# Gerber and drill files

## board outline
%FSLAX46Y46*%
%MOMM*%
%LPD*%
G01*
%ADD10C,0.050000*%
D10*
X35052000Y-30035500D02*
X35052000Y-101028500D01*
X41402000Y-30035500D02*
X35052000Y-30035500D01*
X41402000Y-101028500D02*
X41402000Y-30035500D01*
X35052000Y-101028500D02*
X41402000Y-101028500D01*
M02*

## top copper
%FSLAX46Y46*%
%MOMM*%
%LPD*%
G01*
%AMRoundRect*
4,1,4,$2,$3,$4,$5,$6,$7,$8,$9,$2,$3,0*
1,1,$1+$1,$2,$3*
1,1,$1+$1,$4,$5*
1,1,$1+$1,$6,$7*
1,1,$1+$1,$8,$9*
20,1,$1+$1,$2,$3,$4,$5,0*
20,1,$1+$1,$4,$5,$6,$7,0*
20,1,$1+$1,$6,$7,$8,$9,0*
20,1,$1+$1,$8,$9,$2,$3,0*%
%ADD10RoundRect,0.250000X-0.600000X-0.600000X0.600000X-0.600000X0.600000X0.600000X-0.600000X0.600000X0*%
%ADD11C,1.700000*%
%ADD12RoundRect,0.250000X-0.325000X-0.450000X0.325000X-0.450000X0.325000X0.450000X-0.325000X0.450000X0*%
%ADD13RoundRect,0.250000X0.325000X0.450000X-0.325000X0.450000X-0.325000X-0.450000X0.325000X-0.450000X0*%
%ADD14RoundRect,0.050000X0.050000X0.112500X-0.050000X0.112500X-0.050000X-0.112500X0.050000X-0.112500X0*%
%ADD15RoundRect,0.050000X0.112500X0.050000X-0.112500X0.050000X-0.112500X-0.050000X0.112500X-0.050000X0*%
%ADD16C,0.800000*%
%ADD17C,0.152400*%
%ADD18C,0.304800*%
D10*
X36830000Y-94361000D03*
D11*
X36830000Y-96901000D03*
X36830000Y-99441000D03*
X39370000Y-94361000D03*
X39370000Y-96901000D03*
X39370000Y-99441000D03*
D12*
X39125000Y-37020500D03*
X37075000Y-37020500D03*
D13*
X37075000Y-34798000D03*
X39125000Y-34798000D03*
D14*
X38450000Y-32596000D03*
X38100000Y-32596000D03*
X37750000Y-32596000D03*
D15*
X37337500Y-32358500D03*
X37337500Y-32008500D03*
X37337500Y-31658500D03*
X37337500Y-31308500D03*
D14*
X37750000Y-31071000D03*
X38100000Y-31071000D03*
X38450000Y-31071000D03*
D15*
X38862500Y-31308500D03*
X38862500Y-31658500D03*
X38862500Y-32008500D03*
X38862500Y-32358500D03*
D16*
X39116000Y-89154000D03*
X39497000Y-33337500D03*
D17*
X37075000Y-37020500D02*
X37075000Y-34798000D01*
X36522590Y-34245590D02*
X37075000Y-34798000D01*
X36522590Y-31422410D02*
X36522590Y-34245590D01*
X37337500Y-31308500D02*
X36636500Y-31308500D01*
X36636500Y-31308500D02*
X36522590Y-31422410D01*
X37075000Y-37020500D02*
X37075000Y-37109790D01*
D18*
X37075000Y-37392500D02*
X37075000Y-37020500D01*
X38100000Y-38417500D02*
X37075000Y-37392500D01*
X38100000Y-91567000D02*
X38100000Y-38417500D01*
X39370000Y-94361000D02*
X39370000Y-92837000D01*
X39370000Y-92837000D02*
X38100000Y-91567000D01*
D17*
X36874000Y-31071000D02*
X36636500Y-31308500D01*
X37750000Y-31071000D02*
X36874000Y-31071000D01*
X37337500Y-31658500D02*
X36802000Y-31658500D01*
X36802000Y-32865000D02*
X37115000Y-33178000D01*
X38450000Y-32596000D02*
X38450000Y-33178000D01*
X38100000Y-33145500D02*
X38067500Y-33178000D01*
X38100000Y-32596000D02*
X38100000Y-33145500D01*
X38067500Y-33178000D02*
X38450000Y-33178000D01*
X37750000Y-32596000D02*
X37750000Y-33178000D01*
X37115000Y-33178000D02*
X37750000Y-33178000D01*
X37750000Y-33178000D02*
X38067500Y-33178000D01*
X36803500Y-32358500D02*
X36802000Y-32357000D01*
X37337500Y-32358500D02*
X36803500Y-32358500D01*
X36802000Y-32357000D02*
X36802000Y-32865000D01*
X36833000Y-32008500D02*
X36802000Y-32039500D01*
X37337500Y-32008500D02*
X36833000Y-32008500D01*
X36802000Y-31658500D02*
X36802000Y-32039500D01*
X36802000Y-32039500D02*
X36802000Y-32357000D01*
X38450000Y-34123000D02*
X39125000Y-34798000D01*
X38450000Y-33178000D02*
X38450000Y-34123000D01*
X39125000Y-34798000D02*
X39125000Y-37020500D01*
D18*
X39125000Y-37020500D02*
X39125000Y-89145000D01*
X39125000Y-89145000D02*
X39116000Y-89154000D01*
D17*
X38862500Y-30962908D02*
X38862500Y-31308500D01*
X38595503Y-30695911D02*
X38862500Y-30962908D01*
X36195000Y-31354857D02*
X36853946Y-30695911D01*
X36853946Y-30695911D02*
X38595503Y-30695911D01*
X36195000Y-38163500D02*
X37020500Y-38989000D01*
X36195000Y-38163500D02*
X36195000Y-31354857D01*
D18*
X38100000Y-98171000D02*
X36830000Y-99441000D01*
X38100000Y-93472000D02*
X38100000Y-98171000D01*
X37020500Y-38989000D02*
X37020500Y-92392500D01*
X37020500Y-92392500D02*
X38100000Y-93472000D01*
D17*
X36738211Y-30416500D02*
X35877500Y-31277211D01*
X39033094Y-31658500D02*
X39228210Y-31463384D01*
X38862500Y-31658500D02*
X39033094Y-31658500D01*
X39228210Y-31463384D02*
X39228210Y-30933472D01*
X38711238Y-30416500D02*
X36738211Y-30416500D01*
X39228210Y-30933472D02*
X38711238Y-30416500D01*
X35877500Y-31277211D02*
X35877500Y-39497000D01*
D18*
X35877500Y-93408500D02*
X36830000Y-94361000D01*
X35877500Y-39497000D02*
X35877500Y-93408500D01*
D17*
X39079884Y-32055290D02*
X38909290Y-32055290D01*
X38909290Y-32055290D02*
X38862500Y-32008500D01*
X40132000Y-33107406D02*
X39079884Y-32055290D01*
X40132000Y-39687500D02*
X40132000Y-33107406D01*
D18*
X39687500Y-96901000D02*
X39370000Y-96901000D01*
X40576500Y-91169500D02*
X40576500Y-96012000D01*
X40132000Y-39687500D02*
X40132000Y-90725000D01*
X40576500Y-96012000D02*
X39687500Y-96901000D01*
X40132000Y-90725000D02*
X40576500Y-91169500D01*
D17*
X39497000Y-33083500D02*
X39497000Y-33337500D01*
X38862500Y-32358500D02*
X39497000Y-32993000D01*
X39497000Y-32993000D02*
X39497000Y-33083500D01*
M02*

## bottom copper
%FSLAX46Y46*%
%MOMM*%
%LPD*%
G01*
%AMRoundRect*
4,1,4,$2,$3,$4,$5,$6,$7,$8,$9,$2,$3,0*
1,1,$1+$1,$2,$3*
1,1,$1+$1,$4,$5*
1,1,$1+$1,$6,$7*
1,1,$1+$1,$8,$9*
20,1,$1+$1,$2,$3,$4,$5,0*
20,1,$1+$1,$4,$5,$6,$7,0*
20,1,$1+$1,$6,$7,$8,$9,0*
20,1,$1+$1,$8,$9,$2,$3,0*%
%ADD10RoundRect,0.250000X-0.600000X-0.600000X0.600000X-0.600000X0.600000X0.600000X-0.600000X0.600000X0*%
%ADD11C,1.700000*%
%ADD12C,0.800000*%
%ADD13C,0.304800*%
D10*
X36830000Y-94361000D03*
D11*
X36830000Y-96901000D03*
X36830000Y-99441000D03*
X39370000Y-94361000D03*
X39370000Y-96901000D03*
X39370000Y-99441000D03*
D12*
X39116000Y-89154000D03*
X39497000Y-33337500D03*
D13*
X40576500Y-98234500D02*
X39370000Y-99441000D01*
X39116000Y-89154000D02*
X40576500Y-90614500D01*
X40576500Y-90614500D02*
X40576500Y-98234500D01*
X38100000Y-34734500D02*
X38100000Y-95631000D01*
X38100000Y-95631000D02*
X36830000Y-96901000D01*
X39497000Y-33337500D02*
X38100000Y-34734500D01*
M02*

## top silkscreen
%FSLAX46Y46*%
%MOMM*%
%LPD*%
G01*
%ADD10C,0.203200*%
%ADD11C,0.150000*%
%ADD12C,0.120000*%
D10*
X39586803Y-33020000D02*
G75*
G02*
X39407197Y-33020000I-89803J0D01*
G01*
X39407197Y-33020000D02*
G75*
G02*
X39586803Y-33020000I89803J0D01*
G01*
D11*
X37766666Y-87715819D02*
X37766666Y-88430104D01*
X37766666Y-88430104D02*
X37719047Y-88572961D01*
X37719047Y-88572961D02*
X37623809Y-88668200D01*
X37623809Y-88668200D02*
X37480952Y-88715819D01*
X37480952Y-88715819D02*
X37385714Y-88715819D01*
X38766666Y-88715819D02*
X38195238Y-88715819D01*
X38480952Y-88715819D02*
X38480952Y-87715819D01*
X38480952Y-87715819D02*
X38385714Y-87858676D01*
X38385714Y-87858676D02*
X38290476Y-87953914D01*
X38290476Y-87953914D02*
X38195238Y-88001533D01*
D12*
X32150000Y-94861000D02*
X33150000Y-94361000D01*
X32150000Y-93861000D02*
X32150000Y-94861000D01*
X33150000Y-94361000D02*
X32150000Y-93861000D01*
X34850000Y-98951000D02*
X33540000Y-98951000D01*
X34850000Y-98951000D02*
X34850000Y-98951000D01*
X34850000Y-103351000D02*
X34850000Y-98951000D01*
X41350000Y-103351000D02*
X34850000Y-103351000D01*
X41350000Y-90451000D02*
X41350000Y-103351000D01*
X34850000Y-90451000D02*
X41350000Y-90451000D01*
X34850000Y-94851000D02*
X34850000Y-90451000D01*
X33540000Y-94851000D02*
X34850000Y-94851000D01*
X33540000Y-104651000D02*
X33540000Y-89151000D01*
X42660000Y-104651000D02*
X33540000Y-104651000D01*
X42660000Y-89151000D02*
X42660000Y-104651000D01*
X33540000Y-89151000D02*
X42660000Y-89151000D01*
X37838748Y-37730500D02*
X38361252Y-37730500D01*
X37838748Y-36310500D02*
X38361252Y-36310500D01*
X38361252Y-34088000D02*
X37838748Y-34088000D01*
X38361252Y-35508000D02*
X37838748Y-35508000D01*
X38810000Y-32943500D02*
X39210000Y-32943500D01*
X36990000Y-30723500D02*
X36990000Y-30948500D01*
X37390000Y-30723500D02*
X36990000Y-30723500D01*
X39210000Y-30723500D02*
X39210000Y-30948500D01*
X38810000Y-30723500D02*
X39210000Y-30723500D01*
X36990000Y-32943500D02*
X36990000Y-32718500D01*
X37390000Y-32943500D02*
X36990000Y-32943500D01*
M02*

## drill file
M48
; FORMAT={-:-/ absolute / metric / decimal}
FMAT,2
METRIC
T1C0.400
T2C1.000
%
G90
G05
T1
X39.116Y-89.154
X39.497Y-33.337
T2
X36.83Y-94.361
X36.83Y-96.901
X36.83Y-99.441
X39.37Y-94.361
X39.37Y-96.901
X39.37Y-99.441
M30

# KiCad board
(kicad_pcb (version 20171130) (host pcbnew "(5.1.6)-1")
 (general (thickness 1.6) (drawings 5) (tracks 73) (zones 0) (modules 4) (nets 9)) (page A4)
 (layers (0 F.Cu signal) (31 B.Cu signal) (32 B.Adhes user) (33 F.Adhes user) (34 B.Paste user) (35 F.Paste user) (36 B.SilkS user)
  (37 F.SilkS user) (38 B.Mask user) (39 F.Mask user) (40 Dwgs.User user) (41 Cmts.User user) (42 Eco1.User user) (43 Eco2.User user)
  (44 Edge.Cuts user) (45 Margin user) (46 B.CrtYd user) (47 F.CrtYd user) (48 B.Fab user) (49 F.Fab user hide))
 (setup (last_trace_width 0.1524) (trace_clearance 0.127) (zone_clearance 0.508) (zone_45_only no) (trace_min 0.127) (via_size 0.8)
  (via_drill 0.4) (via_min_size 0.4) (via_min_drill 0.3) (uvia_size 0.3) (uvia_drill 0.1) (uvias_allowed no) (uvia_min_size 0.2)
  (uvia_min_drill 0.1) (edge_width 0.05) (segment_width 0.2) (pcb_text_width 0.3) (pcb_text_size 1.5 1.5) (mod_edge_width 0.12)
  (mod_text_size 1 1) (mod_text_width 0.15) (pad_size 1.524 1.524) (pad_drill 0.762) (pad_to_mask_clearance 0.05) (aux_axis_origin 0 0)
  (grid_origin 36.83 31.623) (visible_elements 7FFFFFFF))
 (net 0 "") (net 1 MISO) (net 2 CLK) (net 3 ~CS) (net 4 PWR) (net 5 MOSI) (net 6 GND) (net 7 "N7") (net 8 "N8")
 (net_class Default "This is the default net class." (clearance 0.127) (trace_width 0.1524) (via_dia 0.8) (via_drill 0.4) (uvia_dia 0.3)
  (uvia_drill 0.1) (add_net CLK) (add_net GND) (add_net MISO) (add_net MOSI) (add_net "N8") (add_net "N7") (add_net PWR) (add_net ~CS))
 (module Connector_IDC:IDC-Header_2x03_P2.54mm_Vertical (layer F.Cu) (at 36.83 94.361)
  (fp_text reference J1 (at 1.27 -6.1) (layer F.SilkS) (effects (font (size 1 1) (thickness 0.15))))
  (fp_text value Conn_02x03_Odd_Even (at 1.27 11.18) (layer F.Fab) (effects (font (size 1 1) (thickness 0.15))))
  (fp_line (start -4.68 0.5) (end -3.68 0) (layer F.SilkS) (width 0.12))
  (fp_line (start -4.68 -0.5) (end -4.68 0.5) (layer F.SilkS) (width 0.12))
  (fp_line (start -3.68 0) (end -4.68 -0.5) (layer F.SilkS) (width 0.12))
  (fp_line (start -1.98 4.59) (end -3.29 4.59) (layer F.SilkS) (width 0.12))
  (fp_line (start -1.98 4.59) (end -1.98 4.59) (layer F.SilkS) (width 0.12))
  (fp_line (start -1.98 8.99) (end -1.98 4.59) (layer F.SilkS) (width 0.12))
  (fp_line (start 4.52 8.99) (end -1.98 8.99) (layer F.SilkS) (width 0.12))
  (fp_line (start 4.52 -3.91) (end 4.52 8.99) (layer F.SilkS) (width 0.12))
  (fp_line (start -1.98 -3.91) (end 4.52 -3.91) (layer F.SilkS) (width 0.12))
  (fp_line (start -1.98 0.49) (end -1.98 -3.91) (layer F.SilkS) (width 0.12))
  (fp_line (start -3.29 0.49) (end -1.98 0.49) (layer F.SilkS) (width 0.12))
  (fp_line (start -3.29 10.29) (end -3.29 -5.21) (layer F.SilkS) (width 0.12))
  (fp_line (start 5.83 10.29) (end -3.29 10.29) (layer F.SilkS) (width 0.12))
  (fp_line (start 5.83 -5.21) (end 5.83 10.29) (layer F.SilkS) (width 0.12))
  (fp_line (start -3.29 -5.21) (end 5.83 -5.21) (layer F.SilkS) (width 0.12))
  (pad 1 thru_hole roundrect (at 0 0) (size 1.7 1.7) (drill 1) (layers *.Cu *.Mask) (roundrect_rratio 0.147059) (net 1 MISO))
  (pad 3 thru_hole circle (at 0 2.54) (size 1.7 1.7) (drill 1) (layers *.Cu *.Mask) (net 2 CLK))
  (pad 5 thru_hole circle (at 0 5.08) (size 1.7 1.7) (drill 1) (layers *.Cu *.Mask) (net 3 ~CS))
  (pad 2 thru_hole circle (at 2.54 0) (size 1.7 1.7) (drill 1) (layers *.Cu *.Mask) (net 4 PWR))
  (pad 4 thru_hole circle (at 2.54 2.54) (size 1.7 1.7) (drill 1) (layers *.Cu *.Mask) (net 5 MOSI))
  (pad 6 thru_hole circle (at 2.54 5.08) (size 1.7 1.7) (drill 1) (layers *.Cu *.Mask) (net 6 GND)))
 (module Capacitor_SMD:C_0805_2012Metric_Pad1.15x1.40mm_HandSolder (layer F.Cu) (at 38.1 37.0205)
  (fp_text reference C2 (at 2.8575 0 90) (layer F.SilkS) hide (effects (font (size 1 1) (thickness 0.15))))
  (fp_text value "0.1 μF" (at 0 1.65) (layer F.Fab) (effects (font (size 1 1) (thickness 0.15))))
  (fp_line (start -0.261252 0.71) (end 0.261252 0.71) (layer F.SilkS) (width 0.12))
  (fp_line (start -0.261252 -0.71) (end 0.261252 -0.71) (layer F.SilkS) (width 0.12))
  (pad 2 smd roundrect (at 1.025 0) (size 1.15 1.4) (layers F.Cu F.Paste F.Mask) (roundrect_rratio 0.217391) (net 6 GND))
  (pad 1 smd roundrect (at -1.025 0) (size 1.15 1.4) (layers F.Cu F.Paste F.Mask) (roundrect_rratio 0.217391) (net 4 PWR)))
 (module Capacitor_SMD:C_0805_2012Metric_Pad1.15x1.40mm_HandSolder (layer F.Cu) (at 38.1 34.798 180)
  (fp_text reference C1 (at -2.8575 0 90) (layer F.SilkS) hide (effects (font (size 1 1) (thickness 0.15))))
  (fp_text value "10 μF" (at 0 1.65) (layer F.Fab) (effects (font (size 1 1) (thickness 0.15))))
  (fp_line (start -0.261252 0.71) (end 0.261252 0.71) (layer F.SilkS) (width 0.12))
  (fp_line (start -0.261252 -0.71) (end 0.261252 -0.71) (layer F.SilkS) (width 0.12))
  (pad 2 smd roundrect (at 1.025 0 180) (size 1.15 1.4) (layers F.Cu F.Paste F.Mask) (roundrect_rratio 0.217391) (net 4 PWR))
  (pad 1 smd roundrect (at -1.025 0 180) (size 1.15 1.4) (layers F.Cu F.Paste F.Mask) (roundrect_rratio 0.217391) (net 6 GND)))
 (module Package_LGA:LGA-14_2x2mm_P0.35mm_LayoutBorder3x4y (layer F.Cu) (at 38.1 31.8335 180)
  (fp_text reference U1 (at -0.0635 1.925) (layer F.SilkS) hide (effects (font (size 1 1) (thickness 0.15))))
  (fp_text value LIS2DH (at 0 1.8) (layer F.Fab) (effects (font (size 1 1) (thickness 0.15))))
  (fp_line (start -0.71 -1.11) (end -1.11 -1.11) (layer F.SilkS) (width 0.12))
  (fp_line (start 1.11 1.11) (end 1.11 0.885) (layer F.SilkS) (width 0.12))
  (fp_line (start 0.71 1.11) (end 1.11 1.11) (layer F.SilkS) (width 0.12))
  (fp_line (start -1.11 1.11) (end -1.11 0.885) (layer F.SilkS) (width 0.12))
  (fp_line (start -0.71 1.11) (end -1.11 1.11) (layer F.SilkS) (width 0.12))
  (fp_line (start 1.11 -1.11) (end 1.11 -0.885) (layer F.SilkS) (width 0.12))
  (fp_line (start 0.71 -1.11) (end 1.11 -1.11) (layer F.SilkS) (width 0.12))
  (pad 14 smd roundrect (at -0.35 -0.7625 180) (size 0.2 0.325) (layers F.Cu F.Paste F.Mask) (roundrect_rratio 0.25) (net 6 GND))
  (pad 13 smd roundrect (at 0 -0.7625 180) (size 0.2 0.325) (layers F.Cu F.Paste F.Mask) (roundrect_rratio 0.25) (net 6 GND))
  (pad 12 smd roundrect (at 0.35 -0.7625 180) (size 0.2 0.325) (layers F.Cu F.Paste F.Mask) (roundrect_rratio 0.25) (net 6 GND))
  (pad 11 smd roundrect (at 0.7625 -0.525 180) (size 0.325 0.2) (layers F.Cu F.Paste F.Mask) (roundrect_rratio 0.25) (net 6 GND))
  (pad 10 smd roundrect (at 0.7625 -0.175 180) (size 0.325 0.2) (layers F.Cu F.Paste F.Mask) (roundrect_rratio 0.25) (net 6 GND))
  (pad 9 smd roundrect (at 0.7625 0.175 180) (size 0.325 0.2) (layers F.Cu F.Paste F.Mask) (roundrect_rratio 0.25) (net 6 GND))
  (pad 8 smd roundrect (at 0.7625 0.525 180) (size 0.325 0.2) (layers F.Cu F.Paste F.Mask) (roundrect_rratio 0.25) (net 4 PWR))
  (pad 7 smd roundrect (at 0.35 0.7625 180) (size 0.2 0.325) (layers F.Cu F.Paste F.Mask) (roundrect_rratio 0.25) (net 4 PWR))
  (pad 6 smd roundrect (at 0 0.7625 180) (size 0.2 0.325) (layers F.Cu F.Paste F.Mask) (roundrect_rratio 0.25) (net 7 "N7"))
  (pad 5 smd roundrect (at -0.35 0.7625 180) (size 0.2 0.325) (layers F.Cu F.Paste F.Mask) (roundrect_rratio 0.25) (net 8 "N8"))
  (pad 4 smd roundrect (at -0.7625 0.525 180) (size 0.325 0.2) (layers F.Cu F.Paste F.Mask) (roundrect_rratio 0.25) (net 3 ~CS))
  (pad 3 smd roundrect (at -0.7625 0.175 180) (size 0.325 0.2) (layers F.Cu F.Paste F.Mask) (roundrect_rratio 0.25) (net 1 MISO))
  (pad 2 smd roundrect (at -0.7625 -0.175 180) (size 0.325 0.2) (layers F.Cu F.Paste F.Mask) (roundrect_rratio 0.25) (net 5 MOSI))
  (pad 1 smd roundrect (at -0.7625 -0.525 180) (size 0.325 0.2) (layers F.Cu F.Paste F.Mask) (roundrect_rratio 0.25) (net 2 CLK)))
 (gr_line (start 35.052 30.0355) (end 35.052 101.0285) (layer Edge.Cuts) (width 0.05))
 (gr_line (start 41.402 30.0355) (end 35.052 30.0355) (layer Edge.Cuts) (width 0.05))
 (gr_line (start 41.402 101.0285) (end 41.402 30.0355) (layer Edge.Cuts) (width 0.05))
 (gr_line (start 35.052 101.0285) (end 41.402 101.0285) (layer Edge.Cuts) (width 0.05))
 (gr_circle (center 39.497 33.02) (end 39.586803 33.02) (layer F.SilkS) (width 0.2032))
 (segment (start 37.075 37.0205) (end 37.075 34.798) (width 0.1524) (layer F.Cu) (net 4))
 (segment (start 36.52259 34.24559) (end 37.075 34.798) (width 0.1524) (layer F.Cu) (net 4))
 (segment (start 36.52259 31.42241) (end 36.52259 34.24559) (width 0.1524) (layer F.Cu) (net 4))
 (segment (start 37.3375 31.3085) (end 36.6365 31.3085) (width 0.1524) (layer F.Cu) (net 4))
 (segment (start 36.6365 31.3085) (end 36.52259 31.42241) (width 0.1524) (layer F.Cu) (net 4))
 (segment (start 37.075 37.0205) (end 37.075 37.10979) (width 0.1524) (layer F.Cu) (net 4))
 (segment (start 37.075 37.3925) (end 37.075 37.0205) (width 0.3048) (layer F.Cu) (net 4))
 (segment (start 38.1 38.4175) (end 37.075 37.3925) (width 0.3048) (layer F.Cu) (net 4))
 (segment (start 38.1 91.567) (end 38.1 38.4175) (width 0.3048) (layer F.Cu) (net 4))
 (segment (start 39.37 94.361) (end 39.37 92.837) (width 0.3048) (layer F.Cu) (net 4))
 (segment (start 39.37 92.837) (end 38.1 91.567) (width 0.3048) (layer F.Cu) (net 4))
 (segment (start 36.874 31.071) (end 36.6365 31.3085) (width 0.1524) (layer F.Cu) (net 4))
 (segment (start 37.75 31.071) (end 36.874 31.071) (width 0.1524) (layer F.Cu) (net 4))
 (segment (start 37.3375 31.6585) (end 36.802 31.6585) (width 0.1524) (layer F.Cu) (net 6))
 (segment (start 36.802 32.865) (end 37.115 33.178) (width 0.1524) (layer F.Cu) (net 6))
 (segment (start 38.45 32.596) (end 38.45 33.178) (width 0.1524) (layer F.Cu) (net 6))
 (segment (start 38.1 33.1455) (end 38.0675 33.178) (width 0.1524) (layer F.Cu) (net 6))
 (segment (start 38.1 32.596) (end 38.1 33.1455) (width 0.1524) (layer F.Cu) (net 6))
 (segment (start 38.0675 33.178) (end 38.45 33.178) (width 0.1524) (layer F.Cu) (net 6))
 (segment (start 37.75 32.596) (end 37.75 33.178) (width 0.1524) (layer F.Cu) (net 6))
 (segment (start 37.115 33.178) (end 37.75 33.178) (width 0.1524) (layer F.Cu) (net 6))
 (segment (start 37.75 33.178) (end 38.0675 33.178) (width 0.1524) (layer F.Cu) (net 6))
 (segment (start 36.8035 32.3585) (end 36.802 32.357) (width 0.1524) (layer F.Cu) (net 6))
 (segment (start 37.3375 32.3585) (end 36.8035 32.3585) (width 0.1524) (layer F.Cu) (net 6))
 (segment (start 36.802 32.357) (end 36.802 32.865) (width 0.1524) (layer F.Cu) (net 6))
 (segment (start 36.833 32.0085) (end 36.802 32.0395) (width 0.1524) (layer F.Cu) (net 6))
 (segment (start 37.3375 32.0085) (end 36.833 32.0085) (width 0.1524) (layer F.Cu) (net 6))
 (segment (start 36.802 31.6585) (end 36.802 32.0395) (width 0.1524) (layer F.Cu) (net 6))
 (segment (start 36.802 32.0395) (end 36.802 32.357) (width 0.1524) (layer F.Cu) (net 6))
 (segment (start 38.45 34.123) (end 39.125 34.798) (width 0.1524) (layer F.Cu) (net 6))
 (segment (start 38.45 33.178) (end 38.45 34.123) (width 0.1524) (layer F.Cu) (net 6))
 (segment (start 39.125 34.798) (end 39.125 37.0205) (width 0.1524) (layer F.Cu) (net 6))
 (segment (start 39.125 37.0205) (end 39.125 89.145) (width 0.3048) (layer F.Cu) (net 6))
 (segment (start 39.125 89.145) (end 39.116 89.154) (width 0.3048) (layer F.Cu) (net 6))
 (via (at 39.116 89.154) (size 0.8) (drill 0.4) (layers F.Cu B.Cu) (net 6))
 (segment (start 40.5765 98.2345) (end 39.37 99.441) (width 0.3048) (layer B.Cu) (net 6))
 (segment (start 39.116 89.154) (end 40.5765 90.6145) (width 0.3048) (layer B.Cu) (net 6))
 (segment (start 40.5765 90.6145) (end 40.5765 98.2345) (width 0.3048) (layer B.Cu) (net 6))
 (segment (start 38.8625 30.962908) (end 38.8625 31.3085) (width 0.1524) (layer F.Cu) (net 3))
 (segment (start 38.595503 30.695911) (end 38.8625 30.962908) (width 0.1524) (layer F.Cu) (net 3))
 (segment (start 36.195 31.354857) (end 36.853946 30.695911) (width 0.1524) (layer F.Cu) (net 3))
 (segment (start 36.853946 30.695911) (end 38.595503 30.695911) (width 0.1524) (layer F.Cu) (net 3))
 (segment (start 36.195 38.1635) (end 37.0205 38.989) (width 0.1524) (layer F.Cu) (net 3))
 (segment (start 36.195 38.1635) (end 36.195 31.354857) (width 0.1524) (layer F.Cu) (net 3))
 (segment (start 38.1 98.171) (end 36.83 99.441) (width 0.3048) (layer F.Cu) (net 3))
 (segment (start 38.1 93.472) (end 38.1 98.171) (width 0.3048) (layer F.Cu) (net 3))
 (segment (start 37.0205 38.989) (end 37.0205 92.3925) (width 0.3048) (layer F.Cu) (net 3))
 (segment (start 37.0205 92.3925) (end 38.1 93.472) (width 0.3048) (layer F.Cu) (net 3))
 (segment (start 36.738211 30.4165) (end 35.8775 31.277211) (width 0.1524) (layer F.Cu) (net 1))
 (segment (start 39.033094 31.6585) (end 39.22821 31.463384) (width 0.1524) (layer F.Cu) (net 1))
 (segment (start 38.8625 31.6585) (end 39.033094 31.6585) (width 0.1524) (layer F.Cu) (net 1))
 (segment (start 39.22821 31.463384) (end 39.22821 30.933472) (width 0.1524) (layer F.Cu) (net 1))
 (segment (start 38.711238 30.4165) (end 36.738211 30.4165) (width 0.1524) (layer F.Cu) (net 1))
 (segment (start 39.22821 30.933472) (end 38.711238 30.4165) (width 0.1524) (layer F.Cu) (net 1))
 (segment (start 35.8775 31.277211) (end 35.8775 39.497) (width 0.1524) (layer F.Cu) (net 1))
 (segment (start 35.8775 93.4085) (end 36.83 94.361) (width 0.3048) (layer F.Cu) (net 1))
 (segment (start 35.8775 39.497) (end 35.8775 93.4085) (width 0.3048) (layer F.Cu) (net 1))
 (segment (start 39.079884 32.05529) (end 38.90929 32.05529) (width 0.1524) (layer F.Cu) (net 5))
 (segment (start 38.90929 32.05529) (end 38.8625 32.0085) (width 0.1524) (layer F.Cu) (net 5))
 (segment (start 40.132 33.107406) (end 39.079884 32.05529) (width 0.1524) (layer F.Cu) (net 5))
 (segment (start 40.132 39.6875) (end 40.132 33.107406) (width 0.1524) (layer F.Cu) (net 5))
 (segment (start 39.6875 96.901) (end 39.37 96.901) (width 0.3048) (layer F.Cu) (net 5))
 (segment (start 40.5765 91.1695) (end 40.5765 96.012) (width 0.3048) (layer F.Cu) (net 5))
 (segment (start 40.132 39.6875) (end 40.132 90.725) (width 0.3048) (layer F.Cu) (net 5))
 (segment (start 40.5765 96.012) (end 39.6875 96.901) (width 0.3048) (layer F.Cu) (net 5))
 (segment (start 40.132 90.725) (end 40.5765 91.1695) (width 0.3048) (layer F.Cu) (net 5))
 (segment (start 38.1 34.7345) (end 38.1 95.631) (width 0.3048) (layer B.Cu) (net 2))
 (segment (start 38.1 95.631) (end 36.83 96.901) (width 0.3048) (layer B.Cu) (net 2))
 (segment (start 39.497 33.3375) (end 38.1 34.7345) (width 0.3048) (layer B.Cu) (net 2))
 (segment (start 39.497 33.0835) (end 39.497 33.3375) (width 0.1524) (layer F.Cu) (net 2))
 (via (at 39.497 33.3375) (size 0.8) (drill 0.4) (layers F.Cu B.Cu) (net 2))
 (segment (start 38.8625 32.3585) (end 39.497 32.993) (width 0.1524) (layer F.Cu) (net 2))
 (segment (start 39.497 32.993) (end 39.497 33.0835) (width 0.1524) (layer F.Cu) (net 2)))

